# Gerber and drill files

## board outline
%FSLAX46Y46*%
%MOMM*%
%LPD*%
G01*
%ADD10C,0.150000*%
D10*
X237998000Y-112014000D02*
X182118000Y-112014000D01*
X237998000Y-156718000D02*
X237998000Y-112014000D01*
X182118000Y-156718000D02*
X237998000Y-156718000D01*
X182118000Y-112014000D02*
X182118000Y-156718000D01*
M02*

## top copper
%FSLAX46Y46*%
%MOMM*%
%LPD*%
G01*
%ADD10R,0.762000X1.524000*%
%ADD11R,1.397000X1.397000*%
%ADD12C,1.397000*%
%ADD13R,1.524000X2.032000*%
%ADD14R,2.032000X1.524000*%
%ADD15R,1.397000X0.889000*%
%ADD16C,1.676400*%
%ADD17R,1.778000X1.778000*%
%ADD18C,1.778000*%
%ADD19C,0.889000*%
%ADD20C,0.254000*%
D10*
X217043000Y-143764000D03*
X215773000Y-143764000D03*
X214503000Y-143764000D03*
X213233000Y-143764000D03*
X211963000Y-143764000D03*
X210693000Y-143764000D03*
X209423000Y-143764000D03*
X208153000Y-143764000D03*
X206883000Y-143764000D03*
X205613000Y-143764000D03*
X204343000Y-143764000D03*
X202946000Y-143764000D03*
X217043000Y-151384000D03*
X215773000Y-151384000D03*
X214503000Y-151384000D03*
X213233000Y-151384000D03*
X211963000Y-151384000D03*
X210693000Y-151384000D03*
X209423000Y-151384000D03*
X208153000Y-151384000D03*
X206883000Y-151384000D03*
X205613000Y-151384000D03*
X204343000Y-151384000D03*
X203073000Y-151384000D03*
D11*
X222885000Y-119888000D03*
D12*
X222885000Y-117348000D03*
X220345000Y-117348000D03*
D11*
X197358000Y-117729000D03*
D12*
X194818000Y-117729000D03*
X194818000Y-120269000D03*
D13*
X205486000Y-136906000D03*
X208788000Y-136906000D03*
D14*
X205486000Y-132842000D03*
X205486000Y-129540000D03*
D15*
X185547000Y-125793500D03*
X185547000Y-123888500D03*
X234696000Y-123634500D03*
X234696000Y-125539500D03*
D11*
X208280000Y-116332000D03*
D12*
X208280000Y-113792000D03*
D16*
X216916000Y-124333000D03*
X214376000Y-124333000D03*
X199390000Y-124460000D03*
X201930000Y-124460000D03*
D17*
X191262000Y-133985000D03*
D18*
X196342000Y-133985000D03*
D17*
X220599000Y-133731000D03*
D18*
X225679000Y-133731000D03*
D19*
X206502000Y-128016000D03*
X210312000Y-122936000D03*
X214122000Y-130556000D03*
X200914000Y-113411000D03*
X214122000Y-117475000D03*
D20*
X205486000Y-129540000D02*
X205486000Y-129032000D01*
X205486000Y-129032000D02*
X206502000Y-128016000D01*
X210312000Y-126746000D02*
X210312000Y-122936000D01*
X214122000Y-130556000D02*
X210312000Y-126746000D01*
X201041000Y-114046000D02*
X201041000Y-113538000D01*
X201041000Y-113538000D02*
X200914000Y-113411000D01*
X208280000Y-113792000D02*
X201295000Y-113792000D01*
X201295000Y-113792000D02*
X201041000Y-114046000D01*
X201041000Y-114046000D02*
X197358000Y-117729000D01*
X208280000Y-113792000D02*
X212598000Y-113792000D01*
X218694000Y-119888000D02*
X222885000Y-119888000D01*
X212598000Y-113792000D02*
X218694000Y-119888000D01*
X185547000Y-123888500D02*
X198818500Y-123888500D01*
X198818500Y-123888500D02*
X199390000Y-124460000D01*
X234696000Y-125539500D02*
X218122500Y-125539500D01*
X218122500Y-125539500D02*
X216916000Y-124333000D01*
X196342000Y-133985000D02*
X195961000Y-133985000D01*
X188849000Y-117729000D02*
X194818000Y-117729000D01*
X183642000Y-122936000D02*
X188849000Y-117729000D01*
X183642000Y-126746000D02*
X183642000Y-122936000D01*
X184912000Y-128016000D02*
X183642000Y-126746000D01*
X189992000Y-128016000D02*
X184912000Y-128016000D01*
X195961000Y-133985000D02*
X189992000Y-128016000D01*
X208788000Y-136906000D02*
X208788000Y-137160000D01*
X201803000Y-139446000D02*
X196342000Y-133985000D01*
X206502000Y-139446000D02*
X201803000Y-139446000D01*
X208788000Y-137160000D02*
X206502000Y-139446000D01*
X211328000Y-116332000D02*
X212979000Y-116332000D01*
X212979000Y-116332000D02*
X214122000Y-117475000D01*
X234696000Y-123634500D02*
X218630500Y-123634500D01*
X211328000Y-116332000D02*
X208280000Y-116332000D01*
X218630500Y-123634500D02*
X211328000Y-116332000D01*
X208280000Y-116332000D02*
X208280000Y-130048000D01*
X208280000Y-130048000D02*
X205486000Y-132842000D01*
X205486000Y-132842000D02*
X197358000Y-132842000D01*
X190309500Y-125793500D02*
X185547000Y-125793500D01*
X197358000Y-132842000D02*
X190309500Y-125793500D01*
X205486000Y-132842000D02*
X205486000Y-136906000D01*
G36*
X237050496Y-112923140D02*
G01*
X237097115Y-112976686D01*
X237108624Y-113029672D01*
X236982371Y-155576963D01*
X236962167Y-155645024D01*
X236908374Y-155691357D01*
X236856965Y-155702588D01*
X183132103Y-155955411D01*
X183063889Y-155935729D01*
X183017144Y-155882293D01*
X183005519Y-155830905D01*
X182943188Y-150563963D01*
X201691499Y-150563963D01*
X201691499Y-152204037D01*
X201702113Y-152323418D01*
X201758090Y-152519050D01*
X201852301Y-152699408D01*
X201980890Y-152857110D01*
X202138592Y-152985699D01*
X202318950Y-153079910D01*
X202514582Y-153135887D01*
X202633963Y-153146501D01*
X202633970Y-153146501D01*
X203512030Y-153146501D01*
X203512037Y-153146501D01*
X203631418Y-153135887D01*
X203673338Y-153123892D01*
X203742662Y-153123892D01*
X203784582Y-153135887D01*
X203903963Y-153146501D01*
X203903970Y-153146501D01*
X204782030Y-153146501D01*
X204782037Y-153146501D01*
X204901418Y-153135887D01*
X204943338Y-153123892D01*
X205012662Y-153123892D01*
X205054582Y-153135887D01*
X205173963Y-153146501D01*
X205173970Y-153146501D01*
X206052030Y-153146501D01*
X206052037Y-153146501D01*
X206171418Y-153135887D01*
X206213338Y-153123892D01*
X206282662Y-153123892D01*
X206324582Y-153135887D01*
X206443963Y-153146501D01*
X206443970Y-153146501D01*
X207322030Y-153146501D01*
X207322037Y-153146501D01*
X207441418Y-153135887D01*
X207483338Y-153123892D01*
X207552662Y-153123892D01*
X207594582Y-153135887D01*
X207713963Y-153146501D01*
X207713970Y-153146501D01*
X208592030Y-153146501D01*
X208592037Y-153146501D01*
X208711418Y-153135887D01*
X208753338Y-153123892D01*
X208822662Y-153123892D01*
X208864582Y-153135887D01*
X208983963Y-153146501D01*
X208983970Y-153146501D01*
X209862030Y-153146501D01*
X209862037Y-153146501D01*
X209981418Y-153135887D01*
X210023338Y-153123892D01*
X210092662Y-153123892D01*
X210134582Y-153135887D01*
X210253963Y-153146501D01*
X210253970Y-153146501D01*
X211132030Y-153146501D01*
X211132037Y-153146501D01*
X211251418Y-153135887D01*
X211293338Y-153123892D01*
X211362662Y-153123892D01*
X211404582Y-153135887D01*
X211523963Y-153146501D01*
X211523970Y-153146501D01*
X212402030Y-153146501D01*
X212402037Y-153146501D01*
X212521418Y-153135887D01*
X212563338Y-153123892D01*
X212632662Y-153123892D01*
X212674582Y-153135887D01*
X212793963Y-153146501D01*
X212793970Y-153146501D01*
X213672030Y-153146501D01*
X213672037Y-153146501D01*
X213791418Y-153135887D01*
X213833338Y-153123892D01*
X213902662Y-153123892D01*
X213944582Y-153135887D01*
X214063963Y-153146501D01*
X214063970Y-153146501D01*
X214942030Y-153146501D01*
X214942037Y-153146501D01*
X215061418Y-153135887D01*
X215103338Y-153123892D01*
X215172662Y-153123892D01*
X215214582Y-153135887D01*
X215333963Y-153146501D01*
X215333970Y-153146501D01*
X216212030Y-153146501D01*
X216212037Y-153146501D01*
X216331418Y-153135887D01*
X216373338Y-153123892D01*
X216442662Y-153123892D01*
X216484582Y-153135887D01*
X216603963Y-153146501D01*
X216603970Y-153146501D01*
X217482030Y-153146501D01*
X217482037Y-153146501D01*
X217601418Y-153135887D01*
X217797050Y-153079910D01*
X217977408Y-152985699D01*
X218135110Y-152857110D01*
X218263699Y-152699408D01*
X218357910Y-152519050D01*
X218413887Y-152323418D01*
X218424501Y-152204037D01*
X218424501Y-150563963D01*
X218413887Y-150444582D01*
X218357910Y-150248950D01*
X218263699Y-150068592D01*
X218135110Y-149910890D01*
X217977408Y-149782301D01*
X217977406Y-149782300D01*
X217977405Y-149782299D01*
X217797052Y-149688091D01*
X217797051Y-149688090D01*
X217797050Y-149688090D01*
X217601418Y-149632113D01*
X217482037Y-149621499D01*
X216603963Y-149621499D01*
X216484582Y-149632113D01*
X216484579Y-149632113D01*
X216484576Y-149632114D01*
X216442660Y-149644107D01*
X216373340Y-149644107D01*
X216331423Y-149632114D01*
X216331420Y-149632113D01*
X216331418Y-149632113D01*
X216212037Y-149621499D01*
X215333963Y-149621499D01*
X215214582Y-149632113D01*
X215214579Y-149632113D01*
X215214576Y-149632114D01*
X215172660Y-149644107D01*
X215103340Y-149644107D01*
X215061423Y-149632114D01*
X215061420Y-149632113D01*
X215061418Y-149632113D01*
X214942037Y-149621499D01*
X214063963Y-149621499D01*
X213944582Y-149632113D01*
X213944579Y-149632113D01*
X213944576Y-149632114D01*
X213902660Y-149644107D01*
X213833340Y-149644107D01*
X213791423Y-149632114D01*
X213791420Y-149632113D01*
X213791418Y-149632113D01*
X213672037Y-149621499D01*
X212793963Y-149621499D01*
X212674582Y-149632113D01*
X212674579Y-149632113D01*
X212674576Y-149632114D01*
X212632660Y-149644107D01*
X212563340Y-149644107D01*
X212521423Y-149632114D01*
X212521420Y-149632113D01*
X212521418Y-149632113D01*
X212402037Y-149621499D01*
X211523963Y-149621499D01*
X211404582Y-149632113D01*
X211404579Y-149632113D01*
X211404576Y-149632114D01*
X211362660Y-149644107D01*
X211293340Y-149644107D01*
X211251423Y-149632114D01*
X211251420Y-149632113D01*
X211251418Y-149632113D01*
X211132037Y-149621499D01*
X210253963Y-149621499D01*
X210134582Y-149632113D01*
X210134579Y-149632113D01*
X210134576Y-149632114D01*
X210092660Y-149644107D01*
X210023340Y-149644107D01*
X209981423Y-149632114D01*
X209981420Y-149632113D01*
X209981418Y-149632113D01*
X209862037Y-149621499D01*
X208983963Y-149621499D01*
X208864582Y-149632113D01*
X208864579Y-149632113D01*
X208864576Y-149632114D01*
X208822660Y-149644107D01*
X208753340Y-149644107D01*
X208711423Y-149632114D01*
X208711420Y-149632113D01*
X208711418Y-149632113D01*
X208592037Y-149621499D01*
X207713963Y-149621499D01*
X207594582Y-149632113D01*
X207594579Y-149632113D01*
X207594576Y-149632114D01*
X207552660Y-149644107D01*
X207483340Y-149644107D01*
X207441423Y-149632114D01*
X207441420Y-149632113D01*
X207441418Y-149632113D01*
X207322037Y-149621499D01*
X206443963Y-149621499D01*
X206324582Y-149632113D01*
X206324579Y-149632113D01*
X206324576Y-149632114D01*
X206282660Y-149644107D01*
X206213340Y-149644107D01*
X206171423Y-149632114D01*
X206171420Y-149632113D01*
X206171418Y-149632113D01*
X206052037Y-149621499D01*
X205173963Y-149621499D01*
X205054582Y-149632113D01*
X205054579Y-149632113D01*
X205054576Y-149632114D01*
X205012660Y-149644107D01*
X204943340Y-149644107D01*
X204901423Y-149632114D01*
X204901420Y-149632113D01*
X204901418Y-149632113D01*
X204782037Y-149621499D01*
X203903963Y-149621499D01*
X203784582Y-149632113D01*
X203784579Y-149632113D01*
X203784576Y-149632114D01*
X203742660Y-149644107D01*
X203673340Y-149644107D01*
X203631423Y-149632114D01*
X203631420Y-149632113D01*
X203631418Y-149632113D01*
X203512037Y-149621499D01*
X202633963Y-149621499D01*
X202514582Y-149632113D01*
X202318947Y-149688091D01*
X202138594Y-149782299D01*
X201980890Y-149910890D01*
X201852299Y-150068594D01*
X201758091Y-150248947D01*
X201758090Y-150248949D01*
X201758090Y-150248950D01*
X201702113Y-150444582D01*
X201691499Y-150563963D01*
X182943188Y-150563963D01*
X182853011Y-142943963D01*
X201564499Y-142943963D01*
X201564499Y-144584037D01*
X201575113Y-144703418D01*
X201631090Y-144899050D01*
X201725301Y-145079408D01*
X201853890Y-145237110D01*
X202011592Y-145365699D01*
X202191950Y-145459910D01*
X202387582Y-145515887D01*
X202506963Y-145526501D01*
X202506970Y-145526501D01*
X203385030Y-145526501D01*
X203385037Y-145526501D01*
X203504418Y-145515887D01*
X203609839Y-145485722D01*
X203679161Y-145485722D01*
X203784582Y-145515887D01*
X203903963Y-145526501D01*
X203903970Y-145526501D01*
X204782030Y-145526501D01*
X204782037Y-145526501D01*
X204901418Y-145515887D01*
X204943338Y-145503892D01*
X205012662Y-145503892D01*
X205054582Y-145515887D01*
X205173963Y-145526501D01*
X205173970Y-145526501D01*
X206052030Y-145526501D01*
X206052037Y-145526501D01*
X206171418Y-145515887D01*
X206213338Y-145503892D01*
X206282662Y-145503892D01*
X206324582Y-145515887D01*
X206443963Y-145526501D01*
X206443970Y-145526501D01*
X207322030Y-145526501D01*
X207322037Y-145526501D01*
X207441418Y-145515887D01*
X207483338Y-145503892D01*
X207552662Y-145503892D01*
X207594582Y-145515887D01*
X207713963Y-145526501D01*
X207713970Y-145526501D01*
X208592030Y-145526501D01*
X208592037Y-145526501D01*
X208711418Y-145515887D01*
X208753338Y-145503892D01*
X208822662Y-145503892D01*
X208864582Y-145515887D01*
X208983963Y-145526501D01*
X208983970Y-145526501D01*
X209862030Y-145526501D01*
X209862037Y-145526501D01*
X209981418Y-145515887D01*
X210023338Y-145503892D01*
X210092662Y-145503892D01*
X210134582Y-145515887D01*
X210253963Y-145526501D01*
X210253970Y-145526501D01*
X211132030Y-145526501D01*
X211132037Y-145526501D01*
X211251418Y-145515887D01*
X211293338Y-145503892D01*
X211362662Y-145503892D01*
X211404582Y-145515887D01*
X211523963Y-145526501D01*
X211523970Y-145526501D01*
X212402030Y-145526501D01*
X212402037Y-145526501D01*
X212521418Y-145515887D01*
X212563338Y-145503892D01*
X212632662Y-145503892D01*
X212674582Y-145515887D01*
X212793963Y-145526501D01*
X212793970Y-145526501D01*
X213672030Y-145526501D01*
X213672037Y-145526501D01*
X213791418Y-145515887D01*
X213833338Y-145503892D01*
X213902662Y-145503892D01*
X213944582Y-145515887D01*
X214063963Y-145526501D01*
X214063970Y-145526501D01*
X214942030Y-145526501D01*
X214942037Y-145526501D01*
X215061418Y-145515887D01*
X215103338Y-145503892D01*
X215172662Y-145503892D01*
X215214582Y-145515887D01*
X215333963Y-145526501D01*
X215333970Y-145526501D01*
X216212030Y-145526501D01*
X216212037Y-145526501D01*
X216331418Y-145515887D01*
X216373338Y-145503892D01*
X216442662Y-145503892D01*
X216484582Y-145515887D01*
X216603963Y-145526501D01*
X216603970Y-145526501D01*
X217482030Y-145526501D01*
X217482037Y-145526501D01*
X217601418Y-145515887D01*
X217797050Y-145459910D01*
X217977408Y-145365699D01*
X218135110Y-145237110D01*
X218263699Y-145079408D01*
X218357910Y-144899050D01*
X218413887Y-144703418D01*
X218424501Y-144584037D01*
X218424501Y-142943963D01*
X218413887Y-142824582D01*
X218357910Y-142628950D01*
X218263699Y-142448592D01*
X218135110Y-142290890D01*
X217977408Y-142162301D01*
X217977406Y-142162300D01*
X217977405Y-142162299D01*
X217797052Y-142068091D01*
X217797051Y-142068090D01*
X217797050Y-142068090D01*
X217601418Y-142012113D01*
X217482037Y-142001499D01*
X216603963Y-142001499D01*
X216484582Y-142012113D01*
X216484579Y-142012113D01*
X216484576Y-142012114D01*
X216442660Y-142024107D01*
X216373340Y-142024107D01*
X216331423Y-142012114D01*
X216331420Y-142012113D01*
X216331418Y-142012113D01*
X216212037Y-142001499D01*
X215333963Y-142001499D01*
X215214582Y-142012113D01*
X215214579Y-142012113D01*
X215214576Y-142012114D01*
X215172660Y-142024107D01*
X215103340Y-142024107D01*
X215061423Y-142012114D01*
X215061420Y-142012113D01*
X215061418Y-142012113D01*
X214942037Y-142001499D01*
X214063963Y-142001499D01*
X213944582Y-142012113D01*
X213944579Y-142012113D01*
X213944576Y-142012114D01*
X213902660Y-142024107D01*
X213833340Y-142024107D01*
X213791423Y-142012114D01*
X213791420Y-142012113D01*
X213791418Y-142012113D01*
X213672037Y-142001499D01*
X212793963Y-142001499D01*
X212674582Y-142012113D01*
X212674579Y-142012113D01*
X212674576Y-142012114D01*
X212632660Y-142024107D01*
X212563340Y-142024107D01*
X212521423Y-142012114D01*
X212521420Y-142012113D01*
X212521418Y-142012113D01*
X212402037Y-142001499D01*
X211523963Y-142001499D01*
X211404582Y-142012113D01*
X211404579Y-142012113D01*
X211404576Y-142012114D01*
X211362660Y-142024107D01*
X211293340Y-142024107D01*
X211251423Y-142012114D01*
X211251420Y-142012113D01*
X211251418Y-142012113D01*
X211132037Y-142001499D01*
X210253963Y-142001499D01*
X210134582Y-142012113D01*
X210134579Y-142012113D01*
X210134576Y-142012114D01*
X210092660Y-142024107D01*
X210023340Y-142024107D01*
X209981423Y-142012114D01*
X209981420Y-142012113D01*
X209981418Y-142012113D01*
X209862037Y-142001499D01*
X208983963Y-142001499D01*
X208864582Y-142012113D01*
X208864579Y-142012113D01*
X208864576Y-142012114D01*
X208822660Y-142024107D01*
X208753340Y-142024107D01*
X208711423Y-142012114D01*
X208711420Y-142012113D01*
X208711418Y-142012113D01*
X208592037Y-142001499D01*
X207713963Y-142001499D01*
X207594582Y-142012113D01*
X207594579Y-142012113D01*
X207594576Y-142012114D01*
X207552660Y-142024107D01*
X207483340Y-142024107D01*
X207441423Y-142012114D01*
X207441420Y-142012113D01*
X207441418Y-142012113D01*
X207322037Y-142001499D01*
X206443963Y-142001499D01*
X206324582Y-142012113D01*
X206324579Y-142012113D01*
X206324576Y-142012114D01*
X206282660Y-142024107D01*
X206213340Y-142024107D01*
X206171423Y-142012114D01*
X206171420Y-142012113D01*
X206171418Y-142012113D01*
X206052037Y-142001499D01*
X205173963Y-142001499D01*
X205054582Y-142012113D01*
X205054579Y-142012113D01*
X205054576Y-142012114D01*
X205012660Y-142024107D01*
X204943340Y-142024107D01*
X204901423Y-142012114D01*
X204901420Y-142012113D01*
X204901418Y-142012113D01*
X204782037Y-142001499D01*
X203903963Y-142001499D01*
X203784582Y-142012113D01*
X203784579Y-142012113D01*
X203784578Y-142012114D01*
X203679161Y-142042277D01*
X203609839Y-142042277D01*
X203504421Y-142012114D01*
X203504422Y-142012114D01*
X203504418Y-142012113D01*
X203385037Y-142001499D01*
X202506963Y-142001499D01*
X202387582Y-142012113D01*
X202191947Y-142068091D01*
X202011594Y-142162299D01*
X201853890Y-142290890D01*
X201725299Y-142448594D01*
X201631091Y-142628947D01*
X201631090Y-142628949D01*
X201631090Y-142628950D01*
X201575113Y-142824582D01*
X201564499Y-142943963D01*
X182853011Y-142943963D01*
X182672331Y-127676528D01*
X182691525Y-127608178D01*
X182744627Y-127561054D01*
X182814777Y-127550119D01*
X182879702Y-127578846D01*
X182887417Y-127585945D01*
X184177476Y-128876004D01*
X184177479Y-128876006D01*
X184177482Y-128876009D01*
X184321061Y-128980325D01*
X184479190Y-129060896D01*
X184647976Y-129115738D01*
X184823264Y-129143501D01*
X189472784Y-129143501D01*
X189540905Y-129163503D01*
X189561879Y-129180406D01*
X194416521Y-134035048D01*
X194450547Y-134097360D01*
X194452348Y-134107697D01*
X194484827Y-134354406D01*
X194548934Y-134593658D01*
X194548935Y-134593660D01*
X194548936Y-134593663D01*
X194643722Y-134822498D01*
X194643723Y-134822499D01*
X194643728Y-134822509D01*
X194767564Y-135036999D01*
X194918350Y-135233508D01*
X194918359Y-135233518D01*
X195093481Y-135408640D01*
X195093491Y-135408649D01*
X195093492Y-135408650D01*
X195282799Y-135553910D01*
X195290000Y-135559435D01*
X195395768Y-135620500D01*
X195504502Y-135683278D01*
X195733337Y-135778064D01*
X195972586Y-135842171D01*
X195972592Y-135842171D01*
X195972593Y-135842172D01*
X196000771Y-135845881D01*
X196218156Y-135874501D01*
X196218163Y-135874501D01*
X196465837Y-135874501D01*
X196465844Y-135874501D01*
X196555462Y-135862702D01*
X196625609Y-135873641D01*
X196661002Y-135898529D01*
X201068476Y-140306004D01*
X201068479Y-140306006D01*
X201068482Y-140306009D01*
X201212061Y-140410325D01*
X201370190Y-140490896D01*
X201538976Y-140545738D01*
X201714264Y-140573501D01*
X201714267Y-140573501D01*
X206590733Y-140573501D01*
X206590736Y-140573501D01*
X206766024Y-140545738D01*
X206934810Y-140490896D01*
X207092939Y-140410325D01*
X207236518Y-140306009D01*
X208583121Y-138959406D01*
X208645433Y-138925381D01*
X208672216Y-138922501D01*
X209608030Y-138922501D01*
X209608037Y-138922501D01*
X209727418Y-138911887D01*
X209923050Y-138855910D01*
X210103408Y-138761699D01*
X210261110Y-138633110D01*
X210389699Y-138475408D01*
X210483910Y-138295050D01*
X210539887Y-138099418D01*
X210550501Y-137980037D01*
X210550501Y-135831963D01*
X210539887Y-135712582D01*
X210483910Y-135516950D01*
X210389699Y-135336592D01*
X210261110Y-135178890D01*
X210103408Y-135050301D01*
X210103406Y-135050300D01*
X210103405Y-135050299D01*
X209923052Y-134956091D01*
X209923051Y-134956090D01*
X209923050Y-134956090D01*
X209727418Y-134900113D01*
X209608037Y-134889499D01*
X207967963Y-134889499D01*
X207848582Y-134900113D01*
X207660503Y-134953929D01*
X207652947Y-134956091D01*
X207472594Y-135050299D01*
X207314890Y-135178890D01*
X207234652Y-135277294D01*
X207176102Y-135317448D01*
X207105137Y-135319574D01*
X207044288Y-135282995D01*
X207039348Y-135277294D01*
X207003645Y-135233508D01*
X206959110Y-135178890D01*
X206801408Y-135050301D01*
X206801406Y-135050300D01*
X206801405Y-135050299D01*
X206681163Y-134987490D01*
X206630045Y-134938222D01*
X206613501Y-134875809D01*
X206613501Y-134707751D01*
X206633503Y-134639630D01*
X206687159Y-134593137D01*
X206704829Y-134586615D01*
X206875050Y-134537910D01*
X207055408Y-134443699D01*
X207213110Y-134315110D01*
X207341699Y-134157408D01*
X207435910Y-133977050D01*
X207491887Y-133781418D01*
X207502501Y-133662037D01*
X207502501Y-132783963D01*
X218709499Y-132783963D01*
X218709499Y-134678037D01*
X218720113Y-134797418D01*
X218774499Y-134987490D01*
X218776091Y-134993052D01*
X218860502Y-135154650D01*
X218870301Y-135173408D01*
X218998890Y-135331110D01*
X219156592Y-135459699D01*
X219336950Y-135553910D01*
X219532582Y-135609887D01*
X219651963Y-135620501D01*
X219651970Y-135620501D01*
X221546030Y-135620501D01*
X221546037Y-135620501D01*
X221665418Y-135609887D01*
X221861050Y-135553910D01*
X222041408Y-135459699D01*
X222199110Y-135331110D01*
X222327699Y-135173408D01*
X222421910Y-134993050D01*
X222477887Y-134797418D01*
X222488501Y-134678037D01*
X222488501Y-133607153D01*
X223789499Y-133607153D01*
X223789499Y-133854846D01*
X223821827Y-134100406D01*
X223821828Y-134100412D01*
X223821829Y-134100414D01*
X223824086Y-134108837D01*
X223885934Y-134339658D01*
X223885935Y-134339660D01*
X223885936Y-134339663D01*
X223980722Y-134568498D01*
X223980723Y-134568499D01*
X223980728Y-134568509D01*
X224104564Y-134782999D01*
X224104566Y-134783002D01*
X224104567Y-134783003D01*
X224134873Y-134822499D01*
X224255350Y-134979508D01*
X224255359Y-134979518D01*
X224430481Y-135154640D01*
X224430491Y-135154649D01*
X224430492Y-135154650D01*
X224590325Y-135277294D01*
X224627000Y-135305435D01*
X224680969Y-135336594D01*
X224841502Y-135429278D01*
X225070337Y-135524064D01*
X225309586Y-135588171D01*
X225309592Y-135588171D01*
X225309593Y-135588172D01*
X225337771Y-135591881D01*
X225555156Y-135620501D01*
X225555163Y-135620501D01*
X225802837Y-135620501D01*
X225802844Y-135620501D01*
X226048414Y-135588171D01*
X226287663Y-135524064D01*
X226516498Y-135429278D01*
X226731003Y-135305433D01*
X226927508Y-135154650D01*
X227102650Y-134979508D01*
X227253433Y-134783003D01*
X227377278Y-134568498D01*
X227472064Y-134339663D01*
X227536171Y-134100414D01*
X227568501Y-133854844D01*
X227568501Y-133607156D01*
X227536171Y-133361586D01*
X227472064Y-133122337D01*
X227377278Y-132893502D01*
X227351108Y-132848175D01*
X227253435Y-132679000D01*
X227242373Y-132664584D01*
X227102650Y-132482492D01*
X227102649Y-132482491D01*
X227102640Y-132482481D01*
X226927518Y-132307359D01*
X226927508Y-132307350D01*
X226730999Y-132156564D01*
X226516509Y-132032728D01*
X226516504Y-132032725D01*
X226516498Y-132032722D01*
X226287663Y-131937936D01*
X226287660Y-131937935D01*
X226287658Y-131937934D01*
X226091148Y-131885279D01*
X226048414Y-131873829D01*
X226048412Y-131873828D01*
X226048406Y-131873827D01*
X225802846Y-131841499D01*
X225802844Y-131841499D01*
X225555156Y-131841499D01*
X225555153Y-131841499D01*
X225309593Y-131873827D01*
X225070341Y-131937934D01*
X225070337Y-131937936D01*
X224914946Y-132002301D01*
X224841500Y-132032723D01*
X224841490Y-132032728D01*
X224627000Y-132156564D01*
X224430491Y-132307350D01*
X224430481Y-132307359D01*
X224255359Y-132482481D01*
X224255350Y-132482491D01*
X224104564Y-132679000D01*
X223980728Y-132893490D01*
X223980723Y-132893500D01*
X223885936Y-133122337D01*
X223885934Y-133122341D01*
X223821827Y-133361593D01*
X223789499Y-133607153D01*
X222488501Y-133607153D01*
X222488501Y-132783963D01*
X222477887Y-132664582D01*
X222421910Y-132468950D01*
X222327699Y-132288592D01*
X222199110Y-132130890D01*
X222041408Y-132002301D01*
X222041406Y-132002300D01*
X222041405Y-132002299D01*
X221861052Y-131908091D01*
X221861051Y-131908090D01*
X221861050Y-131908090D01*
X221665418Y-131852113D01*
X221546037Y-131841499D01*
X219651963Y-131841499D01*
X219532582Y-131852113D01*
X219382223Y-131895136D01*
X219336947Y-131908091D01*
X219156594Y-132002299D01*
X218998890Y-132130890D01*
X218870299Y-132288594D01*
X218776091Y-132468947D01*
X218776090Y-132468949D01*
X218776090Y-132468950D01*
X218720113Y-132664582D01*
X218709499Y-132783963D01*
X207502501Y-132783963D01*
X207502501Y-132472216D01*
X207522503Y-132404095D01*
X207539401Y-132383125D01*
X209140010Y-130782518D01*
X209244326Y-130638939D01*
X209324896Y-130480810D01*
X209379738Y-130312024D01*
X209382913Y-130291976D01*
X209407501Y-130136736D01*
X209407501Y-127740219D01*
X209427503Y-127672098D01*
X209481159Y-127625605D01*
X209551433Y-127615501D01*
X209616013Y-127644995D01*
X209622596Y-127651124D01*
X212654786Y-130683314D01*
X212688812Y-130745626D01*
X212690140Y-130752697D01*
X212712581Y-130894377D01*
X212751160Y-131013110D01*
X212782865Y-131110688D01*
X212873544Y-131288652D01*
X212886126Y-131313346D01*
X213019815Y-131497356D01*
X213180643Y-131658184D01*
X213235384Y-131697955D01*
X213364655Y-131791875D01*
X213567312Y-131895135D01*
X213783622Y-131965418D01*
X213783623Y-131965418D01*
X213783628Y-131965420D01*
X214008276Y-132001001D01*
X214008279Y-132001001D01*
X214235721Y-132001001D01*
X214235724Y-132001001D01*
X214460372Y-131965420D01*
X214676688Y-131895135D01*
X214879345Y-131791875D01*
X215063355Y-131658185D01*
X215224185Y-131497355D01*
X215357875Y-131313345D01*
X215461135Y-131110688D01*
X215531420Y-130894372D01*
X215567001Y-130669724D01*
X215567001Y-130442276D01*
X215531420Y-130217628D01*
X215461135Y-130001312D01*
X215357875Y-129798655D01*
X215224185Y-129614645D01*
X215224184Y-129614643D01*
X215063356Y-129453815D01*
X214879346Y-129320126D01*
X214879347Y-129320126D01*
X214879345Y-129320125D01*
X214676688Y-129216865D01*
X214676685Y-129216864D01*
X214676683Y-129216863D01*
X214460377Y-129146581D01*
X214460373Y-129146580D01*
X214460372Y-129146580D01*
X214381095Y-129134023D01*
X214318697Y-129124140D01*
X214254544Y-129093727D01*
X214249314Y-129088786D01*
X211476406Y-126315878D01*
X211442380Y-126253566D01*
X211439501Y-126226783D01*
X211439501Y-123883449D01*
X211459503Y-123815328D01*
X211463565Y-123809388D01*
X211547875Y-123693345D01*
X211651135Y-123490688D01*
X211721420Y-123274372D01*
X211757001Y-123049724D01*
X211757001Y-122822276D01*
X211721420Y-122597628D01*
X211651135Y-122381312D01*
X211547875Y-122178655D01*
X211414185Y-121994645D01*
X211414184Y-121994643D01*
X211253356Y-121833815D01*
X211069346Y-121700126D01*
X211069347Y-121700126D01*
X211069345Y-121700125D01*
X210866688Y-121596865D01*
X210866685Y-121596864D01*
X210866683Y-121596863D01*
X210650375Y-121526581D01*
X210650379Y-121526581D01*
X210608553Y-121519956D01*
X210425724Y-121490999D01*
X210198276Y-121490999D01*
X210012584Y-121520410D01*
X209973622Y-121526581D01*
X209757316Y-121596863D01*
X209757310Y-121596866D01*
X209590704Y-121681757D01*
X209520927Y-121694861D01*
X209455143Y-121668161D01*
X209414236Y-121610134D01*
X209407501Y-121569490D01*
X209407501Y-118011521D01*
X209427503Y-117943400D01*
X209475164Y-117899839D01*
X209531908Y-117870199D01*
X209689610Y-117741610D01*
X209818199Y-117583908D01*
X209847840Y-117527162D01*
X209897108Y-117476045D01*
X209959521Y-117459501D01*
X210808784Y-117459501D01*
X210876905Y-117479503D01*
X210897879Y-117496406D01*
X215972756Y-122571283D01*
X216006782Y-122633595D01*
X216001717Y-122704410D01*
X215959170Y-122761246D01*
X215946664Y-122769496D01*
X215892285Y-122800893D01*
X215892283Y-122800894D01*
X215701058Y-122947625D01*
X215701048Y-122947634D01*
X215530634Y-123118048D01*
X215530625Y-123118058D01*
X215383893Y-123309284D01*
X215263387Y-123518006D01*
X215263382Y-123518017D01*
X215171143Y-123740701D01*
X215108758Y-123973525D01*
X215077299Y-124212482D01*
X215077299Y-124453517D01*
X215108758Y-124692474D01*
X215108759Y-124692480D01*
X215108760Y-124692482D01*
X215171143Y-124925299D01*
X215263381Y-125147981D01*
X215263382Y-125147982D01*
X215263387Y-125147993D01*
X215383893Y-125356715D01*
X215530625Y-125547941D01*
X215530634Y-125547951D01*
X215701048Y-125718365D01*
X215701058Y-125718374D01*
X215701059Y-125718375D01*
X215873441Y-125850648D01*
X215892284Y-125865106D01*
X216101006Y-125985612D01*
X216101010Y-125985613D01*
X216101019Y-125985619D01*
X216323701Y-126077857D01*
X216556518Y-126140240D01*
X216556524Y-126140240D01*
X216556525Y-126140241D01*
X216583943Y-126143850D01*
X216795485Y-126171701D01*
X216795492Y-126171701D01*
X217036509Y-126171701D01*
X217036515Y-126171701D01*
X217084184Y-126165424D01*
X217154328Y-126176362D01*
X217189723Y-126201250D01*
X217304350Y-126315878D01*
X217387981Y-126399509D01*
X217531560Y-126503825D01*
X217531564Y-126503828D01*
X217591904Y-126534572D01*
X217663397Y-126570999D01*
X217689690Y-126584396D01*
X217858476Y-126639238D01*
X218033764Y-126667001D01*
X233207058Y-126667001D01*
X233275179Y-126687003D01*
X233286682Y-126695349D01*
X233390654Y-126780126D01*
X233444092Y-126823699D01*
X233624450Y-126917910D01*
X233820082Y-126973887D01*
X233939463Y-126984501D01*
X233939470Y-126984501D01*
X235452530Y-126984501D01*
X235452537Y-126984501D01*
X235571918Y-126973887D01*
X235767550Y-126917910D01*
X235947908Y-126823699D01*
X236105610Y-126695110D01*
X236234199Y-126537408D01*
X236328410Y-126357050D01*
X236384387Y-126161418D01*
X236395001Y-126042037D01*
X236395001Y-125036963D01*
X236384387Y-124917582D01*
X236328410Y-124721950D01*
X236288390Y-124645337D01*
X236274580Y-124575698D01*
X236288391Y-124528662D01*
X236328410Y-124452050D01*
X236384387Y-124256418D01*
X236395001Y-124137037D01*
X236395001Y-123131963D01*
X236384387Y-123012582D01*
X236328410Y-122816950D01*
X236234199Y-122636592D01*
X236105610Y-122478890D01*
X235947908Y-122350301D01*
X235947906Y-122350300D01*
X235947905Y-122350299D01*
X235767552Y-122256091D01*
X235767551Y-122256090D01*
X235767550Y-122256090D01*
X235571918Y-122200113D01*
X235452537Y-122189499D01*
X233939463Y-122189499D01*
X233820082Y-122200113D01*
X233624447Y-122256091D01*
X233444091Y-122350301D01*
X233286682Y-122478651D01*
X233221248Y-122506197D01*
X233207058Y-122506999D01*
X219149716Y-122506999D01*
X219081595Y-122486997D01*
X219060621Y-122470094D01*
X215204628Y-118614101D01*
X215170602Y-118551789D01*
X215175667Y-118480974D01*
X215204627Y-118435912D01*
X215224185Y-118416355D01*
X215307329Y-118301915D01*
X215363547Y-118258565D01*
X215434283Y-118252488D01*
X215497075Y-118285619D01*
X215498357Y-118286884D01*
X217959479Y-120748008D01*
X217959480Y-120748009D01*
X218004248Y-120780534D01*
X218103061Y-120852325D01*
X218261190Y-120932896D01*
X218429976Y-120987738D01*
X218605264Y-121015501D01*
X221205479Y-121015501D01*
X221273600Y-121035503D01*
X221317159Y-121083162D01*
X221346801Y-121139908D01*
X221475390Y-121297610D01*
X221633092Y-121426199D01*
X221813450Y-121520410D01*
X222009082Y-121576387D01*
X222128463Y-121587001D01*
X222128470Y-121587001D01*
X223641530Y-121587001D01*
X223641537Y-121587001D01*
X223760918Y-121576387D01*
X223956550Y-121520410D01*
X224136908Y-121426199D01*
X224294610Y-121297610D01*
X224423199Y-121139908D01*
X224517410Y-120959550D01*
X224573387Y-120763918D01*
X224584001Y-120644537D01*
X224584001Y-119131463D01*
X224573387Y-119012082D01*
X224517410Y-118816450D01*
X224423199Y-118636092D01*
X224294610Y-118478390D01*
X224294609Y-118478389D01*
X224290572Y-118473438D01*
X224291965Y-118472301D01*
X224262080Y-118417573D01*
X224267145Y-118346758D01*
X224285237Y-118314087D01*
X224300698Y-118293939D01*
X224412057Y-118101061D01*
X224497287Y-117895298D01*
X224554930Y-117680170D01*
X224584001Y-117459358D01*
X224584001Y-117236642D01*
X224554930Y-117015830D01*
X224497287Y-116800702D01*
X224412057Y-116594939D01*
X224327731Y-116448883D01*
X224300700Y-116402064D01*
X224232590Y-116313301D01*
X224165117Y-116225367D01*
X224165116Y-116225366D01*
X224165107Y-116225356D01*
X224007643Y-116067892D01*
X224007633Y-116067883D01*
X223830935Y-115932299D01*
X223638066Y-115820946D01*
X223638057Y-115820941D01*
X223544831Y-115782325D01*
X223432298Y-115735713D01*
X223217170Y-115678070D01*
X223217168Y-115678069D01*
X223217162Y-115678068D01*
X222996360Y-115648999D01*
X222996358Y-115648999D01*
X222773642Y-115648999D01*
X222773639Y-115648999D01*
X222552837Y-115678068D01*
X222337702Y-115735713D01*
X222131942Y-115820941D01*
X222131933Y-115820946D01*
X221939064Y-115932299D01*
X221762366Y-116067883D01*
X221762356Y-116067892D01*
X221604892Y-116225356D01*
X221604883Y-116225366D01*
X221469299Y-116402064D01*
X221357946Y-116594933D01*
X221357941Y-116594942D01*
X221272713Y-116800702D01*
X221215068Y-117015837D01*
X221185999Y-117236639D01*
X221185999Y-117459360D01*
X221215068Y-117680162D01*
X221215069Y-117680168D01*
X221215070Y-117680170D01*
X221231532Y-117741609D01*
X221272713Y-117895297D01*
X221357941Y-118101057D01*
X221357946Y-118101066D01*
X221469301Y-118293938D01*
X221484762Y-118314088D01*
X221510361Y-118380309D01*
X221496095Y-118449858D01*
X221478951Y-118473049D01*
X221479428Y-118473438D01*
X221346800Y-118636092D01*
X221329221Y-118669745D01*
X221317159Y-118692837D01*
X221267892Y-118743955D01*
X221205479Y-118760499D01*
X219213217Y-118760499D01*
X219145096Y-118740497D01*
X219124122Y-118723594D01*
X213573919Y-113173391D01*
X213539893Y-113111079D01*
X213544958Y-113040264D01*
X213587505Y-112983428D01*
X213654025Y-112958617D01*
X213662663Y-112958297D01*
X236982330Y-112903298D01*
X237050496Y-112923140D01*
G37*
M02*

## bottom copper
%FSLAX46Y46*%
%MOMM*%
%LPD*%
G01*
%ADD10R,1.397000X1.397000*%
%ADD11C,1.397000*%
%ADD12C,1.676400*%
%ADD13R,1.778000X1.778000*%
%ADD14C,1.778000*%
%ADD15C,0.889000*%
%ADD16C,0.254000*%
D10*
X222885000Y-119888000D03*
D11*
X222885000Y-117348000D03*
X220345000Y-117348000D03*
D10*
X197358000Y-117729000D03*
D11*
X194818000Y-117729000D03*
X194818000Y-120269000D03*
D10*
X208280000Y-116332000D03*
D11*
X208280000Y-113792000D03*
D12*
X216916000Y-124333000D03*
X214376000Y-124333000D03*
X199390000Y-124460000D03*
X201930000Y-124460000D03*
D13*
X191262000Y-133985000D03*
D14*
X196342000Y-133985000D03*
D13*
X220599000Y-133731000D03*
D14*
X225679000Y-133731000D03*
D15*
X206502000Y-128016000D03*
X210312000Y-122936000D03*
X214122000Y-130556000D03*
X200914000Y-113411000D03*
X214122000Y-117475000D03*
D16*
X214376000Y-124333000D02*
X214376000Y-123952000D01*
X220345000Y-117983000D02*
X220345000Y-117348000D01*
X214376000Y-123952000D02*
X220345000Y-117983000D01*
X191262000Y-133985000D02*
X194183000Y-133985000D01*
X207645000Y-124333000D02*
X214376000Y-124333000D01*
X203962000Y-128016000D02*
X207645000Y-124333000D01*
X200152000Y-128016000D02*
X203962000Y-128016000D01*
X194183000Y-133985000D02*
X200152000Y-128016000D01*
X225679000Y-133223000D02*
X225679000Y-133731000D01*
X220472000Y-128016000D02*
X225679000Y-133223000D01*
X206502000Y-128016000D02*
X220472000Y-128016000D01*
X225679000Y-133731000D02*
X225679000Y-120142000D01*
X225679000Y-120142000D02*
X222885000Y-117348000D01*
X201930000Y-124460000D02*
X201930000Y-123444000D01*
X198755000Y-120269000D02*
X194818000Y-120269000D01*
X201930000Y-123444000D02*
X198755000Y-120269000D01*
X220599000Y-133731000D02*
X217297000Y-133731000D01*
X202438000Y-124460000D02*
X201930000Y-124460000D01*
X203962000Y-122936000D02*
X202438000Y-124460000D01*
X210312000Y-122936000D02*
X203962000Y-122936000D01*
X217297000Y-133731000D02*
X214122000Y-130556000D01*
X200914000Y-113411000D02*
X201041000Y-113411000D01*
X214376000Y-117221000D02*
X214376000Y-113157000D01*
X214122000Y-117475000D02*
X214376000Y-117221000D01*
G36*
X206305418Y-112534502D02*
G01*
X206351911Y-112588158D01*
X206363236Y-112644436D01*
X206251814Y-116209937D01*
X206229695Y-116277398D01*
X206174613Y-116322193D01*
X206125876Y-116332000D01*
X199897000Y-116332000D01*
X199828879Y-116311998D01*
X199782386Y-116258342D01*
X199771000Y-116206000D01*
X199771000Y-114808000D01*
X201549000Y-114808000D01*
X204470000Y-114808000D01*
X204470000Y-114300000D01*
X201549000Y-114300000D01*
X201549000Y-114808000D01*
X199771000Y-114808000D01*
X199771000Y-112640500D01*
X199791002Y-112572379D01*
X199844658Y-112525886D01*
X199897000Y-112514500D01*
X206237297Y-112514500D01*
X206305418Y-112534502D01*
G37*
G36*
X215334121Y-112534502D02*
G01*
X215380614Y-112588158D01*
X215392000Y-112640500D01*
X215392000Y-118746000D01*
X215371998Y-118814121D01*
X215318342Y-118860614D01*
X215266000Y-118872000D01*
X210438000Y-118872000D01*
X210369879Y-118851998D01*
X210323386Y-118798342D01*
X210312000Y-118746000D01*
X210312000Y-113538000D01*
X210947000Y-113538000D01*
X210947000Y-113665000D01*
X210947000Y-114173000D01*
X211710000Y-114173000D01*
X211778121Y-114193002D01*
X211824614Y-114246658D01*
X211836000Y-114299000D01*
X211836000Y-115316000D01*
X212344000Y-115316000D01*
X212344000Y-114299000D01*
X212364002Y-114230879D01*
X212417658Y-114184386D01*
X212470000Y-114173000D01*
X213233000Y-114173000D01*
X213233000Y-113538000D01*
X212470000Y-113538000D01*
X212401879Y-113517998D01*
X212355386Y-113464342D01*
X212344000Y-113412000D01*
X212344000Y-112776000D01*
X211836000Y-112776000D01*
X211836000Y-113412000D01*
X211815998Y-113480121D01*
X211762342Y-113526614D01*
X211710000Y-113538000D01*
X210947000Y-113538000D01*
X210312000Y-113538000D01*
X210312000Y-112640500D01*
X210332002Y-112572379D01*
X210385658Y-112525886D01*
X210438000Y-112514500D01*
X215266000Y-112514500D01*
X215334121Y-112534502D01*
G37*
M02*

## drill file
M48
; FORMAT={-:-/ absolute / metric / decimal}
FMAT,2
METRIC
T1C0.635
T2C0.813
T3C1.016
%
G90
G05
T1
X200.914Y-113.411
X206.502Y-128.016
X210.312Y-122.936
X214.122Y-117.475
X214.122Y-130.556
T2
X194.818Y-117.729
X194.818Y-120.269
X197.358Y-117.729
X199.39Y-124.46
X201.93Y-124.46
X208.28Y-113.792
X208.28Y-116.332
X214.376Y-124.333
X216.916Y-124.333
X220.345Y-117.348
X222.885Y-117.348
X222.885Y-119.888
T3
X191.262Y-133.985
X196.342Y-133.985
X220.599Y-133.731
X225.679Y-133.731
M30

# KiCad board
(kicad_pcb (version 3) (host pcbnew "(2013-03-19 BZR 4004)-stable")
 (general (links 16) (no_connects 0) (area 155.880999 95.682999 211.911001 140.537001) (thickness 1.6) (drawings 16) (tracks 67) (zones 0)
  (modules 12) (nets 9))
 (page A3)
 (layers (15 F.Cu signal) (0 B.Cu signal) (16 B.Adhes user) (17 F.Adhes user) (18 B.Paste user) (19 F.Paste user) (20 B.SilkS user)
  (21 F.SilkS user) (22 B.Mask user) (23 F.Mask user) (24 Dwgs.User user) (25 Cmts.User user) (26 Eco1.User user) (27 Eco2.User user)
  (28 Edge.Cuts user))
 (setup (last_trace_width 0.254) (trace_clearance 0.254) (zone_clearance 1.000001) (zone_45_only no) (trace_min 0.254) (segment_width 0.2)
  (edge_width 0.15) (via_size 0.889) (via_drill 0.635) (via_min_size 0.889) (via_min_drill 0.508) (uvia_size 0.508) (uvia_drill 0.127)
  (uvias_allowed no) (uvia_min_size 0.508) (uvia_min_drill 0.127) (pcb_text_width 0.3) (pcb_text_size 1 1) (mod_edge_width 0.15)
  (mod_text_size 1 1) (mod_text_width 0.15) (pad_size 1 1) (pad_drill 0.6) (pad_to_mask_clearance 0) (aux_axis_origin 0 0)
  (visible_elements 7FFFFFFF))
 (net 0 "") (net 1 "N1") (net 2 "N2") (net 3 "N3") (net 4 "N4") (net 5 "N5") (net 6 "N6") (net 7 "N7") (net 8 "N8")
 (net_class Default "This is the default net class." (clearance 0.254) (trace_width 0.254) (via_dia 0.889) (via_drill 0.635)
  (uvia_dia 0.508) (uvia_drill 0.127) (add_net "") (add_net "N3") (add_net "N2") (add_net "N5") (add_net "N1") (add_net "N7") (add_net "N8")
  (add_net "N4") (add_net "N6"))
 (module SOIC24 (layer F.Cu) (at 210.058 147.574 180)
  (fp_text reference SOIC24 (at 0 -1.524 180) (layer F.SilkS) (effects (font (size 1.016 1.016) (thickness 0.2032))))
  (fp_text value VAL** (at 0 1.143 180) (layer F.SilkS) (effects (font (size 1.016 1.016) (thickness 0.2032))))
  (pad 1 smd rect (at -6.985 3.81 180) (size 0.762 1.524) (layers F.Cu F.Paste F.Mask))
  (pad 2 smd rect (at -5.715 3.81 180) (size 0.762 1.524) (layers F.Cu F.Paste F.Mask))
  (pad 3 smd rect (at -4.445 3.81 180) (size 0.762 1.524) (layers F.Cu F.Paste F.Mask))
  (pad 4 smd rect (at -3.175 3.81 180) (size 0.762 1.524) (layers F.Cu F.Paste F.Mask))
  (pad 5 smd rect (at -1.905 3.81 180) (size 0.762 1.524) (layers F.Cu F.Paste F.Mask))
  (pad 6 smd rect (at -0.635 3.81 180) (size 0.762 1.524) (layers F.Cu F.Paste F.Mask))
  (pad 7 smd rect (at 0.635 3.81 180) (size 0.762 1.524) (layers F.Cu F.Paste F.Mask))
  (pad 8 smd rect (at 1.905 3.81 180) (size 0.762 1.524) (layers F.Cu F.Paste F.Mask))
  (pad 9 smd rect (at 3.175 3.81 180) (size 0.762 1.524) (layers F.Cu F.Paste F.Mask))
  (pad 10 smd rect (at 4.445 3.81 180) (size 0.762 1.524) (layers F.Cu F.Paste F.Mask))
  (pad 11 smd rect (at 5.715 3.81 180) (size 0.762 1.524) (layers F.Cu F.Paste F.Mask))
  (pad 12 smd rect (at 7.112 3.81 180) (size 0.762 1.524) (layers F.Cu F.Paste F.Mask))
  (pad 24 smd rect (at -6.985 -3.81 180) (size 0.762 1.524) (layers F.Cu F.Paste F.Mask))
  (pad 23 smd rect (at -5.715 -3.81 180) (size 0.762 1.524) (layers F.Cu F.Paste F.Mask))
  (pad 22 smd rect (at -4.445 -3.81 180) (size 0.762 1.524) (layers F.Cu F.Paste F.Mask))
  (pad 21 smd rect (at -3.175 -3.81 180) (size 0.762 1.524) (layers F.Cu F.Paste F.Mask))
  (pad 20 smd rect (at -1.905 -3.81 180) (size 0.762 1.524) (layers F.Cu F.Paste F.Mask))
  (pad 19 smd rect (at -0.635 -3.81 180) (size 0.762 1.524) (layers F.Cu F.Paste F.Mask))
  (pad 18 smd rect (at 0.635 -3.81 180) (size 0.762 1.524) (layers F.Cu F.Paste F.Mask))
  (pad 17 smd rect (at 1.905 -3.81 180) (size 0.762 1.524) (layers F.Cu F.Paste F.Mask))
  (pad 16 smd rect (at 3.175 -3.81 180) (size 0.762 1.524) (layers F.Cu F.Paste F.Mask))
  (pad 15 smd rect (at 4.445 -3.81 180) (size 0.762 1.524) (layers F.Cu F.Paste F.Mask))
  (pad 14 smd rect (at 5.715 -3.81 180) (size 0.762 1.524) (layers F.Cu F.Paste F.Mask))
  (pad 13 smd rect (at 6.985 -3.81 180) (size 0.762 1.524) (layers F.Cu F.Paste F.Mask)))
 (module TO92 (layer F.Cu) (at 221.615 118.618 270) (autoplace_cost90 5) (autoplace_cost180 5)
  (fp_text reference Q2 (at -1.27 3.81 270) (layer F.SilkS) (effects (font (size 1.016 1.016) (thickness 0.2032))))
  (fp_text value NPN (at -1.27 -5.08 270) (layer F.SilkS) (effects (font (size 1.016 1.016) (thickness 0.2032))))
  (pad 1 thru_hole rect (at 1.27 -1.27 270) (size 1.397 1.397) (drill 0.8128) (layers *.Cu *.Mask F.SilkS) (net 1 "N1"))
  (pad 2 thru_hole circle (at -1.27 -1.27 270) (size 1.397 1.397) (drill 0.8128) (layers *.Cu *.Mask F.SilkS) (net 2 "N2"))
  (pad 3 thru_hole circle (at -1.27 1.27 270) (size 1.397 1.397) (drill 0.8128) (layers *.Cu *.Mask F.SilkS) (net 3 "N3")))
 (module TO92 (layer F.Cu) (at 196.088 118.999)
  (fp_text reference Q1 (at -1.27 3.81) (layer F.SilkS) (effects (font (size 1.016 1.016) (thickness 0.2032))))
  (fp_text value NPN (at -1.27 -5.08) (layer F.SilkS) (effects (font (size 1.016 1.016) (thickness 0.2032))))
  (pad 1 thru_hole rect (at 1.27 -1.27) (size 1.397 1.397) (drill 0.8128) (layers *.Cu *.Mask F.SilkS) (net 1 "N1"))
  (pad 2 thru_hole circle (at -1.27 -1.27) (size 1.397 1.397) (drill 0.8128) (layers *.Cu *.Mask F.SilkS) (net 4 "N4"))
  (pad 3 thru_hole circle (at -1.27 1.27) (size 1.397 1.397) (drill 0.8128) (layers *.Cu *.Mask F.SilkS) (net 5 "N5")))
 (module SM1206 (layer F.Cu) (at 207.137 136.906)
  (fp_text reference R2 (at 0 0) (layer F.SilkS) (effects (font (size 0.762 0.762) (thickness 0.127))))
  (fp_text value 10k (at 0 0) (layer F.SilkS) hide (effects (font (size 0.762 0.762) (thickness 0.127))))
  (pad 1 smd rect (at -1.651 0) (size 1.524 2.032) (layers F.Cu F.Paste F.Mask) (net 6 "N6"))
  (pad 2 smd rect (at 1.651 0) (size 1.524 2.032) (layers F.Cu F.Paste F.Mask) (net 4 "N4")))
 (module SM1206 (layer F.Cu) (at 205.486 131.191 90)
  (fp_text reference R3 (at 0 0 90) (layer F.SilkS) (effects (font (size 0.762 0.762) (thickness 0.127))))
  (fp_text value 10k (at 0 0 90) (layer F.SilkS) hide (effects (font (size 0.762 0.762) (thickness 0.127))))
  (pad 1 smd rect (at -1.651 0 90) (size 1.524 2.032) (layers F.Cu F.Paste F.Mask) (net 6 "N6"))
  (pad 2 smd rect (at 1.651 0 90) (size 1.524 2.032) (layers F.Cu F.Paste F.Mask) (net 2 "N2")))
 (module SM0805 (layer F.Cu) (at 185.547 124.841 90)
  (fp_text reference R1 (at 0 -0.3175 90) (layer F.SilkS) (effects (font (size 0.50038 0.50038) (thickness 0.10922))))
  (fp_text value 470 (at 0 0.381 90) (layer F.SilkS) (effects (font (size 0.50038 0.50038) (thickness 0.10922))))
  (pad 1 smd rect (at -0.9525 0 90) (size 0.889 1.397) (layers F.Cu F.Paste F.Mask) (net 6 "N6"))
  (pad 2 smd rect (at 0.9525 0 90) (size 0.889 1.397) (layers F.Cu F.Paste F.Mask) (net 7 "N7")))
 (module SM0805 (layer F.Cu) (at 234.696 124.587 270)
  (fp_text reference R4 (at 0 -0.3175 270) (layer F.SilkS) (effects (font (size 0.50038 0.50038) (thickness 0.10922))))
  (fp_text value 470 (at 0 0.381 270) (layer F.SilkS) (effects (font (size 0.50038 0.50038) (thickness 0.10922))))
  (pad 1 smd rect (at -0.9525 0 270) (size 0.889 1.397) (layers F.Cu F.Paste F.Mask) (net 6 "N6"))
  (pad 2 smd rect (at 0.9525 0 270) (size 0.889 1.397) (layers F.Cu F.Paste F.Mask) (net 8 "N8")))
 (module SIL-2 (layer F.Cu) (at 208.28 115.062 90)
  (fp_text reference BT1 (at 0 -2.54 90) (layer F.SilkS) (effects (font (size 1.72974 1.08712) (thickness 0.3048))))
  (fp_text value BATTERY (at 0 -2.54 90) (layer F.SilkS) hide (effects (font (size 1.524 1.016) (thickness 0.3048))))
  (pad 1 thru_hole rect (at -1.27 0 90) (size 1.397 1.397) (drill 0.8128) (layers *.Cu *.Mask F.SilkS) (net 6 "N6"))
  (pad 2 thru_hole circle (at 1.27 0 90) (size 1.397 1.397) (drill 0.8128) (layers *.Cu *.Mask F.SilkS) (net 1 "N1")))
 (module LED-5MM (layer F.Cu) (at 215.646 124.333 180)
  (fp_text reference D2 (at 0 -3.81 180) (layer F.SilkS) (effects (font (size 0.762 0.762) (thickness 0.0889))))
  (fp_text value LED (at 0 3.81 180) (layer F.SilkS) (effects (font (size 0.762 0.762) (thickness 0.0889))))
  (pad 1 thru_hole circle (at -1.27 0 180) (size 1.6764 1.6764) (drill 0.8128) (layers *.Cu *.Mask F.SilkS) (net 8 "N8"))
  (pad 2 thru_hole circle (at 1.27 0 180) (size 1.6764 1.6764) (drill 0.8128) (layers *.Cu *.Mask F.SilkS) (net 3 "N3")))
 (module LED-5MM (layer F.Cu) (at 200.66 124.46)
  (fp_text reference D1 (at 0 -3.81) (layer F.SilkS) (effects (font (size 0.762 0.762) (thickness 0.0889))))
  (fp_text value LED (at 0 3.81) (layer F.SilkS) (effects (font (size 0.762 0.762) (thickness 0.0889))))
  (pad 1 thru_hole circle (at -1.27 0) (size 1.6764 1.6764) (drill 0.8128) (layers *.Cu *.Mask F.SilkS) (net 7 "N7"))
  (pad 2 thru_hole circle (at 1.27 0) (size 1.6764 1.6764) (drill 0.8128) (layers *.Cu *.Mask F.SilkS) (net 5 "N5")))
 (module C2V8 (layer F.Cu) (at 193.802 133.985)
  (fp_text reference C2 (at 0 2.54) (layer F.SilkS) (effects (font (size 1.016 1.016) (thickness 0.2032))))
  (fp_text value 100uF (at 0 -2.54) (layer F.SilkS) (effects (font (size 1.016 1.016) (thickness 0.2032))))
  (pad 1 thru_hole rect (at -2.54 0) (size 1.778 1.778) (drill 1.016) (layers *.Cu *.Mask F.SilkS) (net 3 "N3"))
  (pad 2 thru_hole circle (at 2.54 0) (size 1.778 1.778) (drill 1.016) (layers *.Cu *.Mask F.SilkS) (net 4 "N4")))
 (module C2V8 (layer F.Cu) (at 223.139 133.731)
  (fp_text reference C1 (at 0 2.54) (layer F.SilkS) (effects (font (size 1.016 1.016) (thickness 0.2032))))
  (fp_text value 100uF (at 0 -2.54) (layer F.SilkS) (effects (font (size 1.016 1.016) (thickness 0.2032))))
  (pad 1 thru_hole rect (at -2.54 0) (size 1.778 1.778) (drill 1.016) (layers *.Cu *.Mask F.SilkS) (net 5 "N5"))
  (pad 2 thru_hole circle (at 2.54 0) (size 1.778 1.778) (drill 1.016) (layers *.Cu *.Mask F.SilkS) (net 2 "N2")))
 (gr_line (start 237.998 112.014) (end 182.118 112.014) (angle 90) (layer Edge.Cuts) (width 0.15))
 (gr_line (start 237.998 156.718) (end 237.998 112.014) (angle 90) (layer Edge.Cuts) (width 0.15))
 (gr_line (start 182.118 156.718) (end 237.998 156.718) (angle 90) (layer Edge.Cuts) (width 0.15))
 (gr_line (start 182.118 112.014) (end 182.118 156.718) (angle 90) (layer Edge.Cuts) (width 0.15))
 (segment (start 214.376 124.333) (end 214.376 123.952) (width 0.254) (layer B.Cu) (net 3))
 (segment (start 220.345 117.983) (end 220.345 117.348) (width 0.254) (layer B.Cu) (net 3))
 (segment (start 214.376 123.952) (end 220.345 117.983) (width 0.254) (layer B.Cu) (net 3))
 (segment (start 191.262 133.985) (end 194.183 133.985) (width 0.254) (layer B.Cu) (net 3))
 (segment (start 207.645 124.333) (end 214.376 124.333) (width 0.254) (layer B.Cu) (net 3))
 (segment (start 203.962 128.016) (end 207.645 124.333) (width 0.254) (layer B.Cu) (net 3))
 (segment (start 200.152 128.016) (end 203.962 128.016) (width 0.254) (layer B.Cu) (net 3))
 (segment (start 194.183 133.985) (end 200.152 128.016) (width 0.254) (layer B.Cu) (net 3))
 (segment (start 205.486 129.54) (end 205.486 129.032) (width 0.254) (layer F.Cu) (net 2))
 (segment (start 225.679 133.223) (end 225.679 133.731) (width 0.254) (layer B.Cu) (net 2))
 (segment (start 220.472 128.016) (end 225.679 133.223) (width 0.254) (layer B.Cu) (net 2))
 (segment (start 206.502 128.016) (end 220.472 128.016) (width 0.254) (layer B.Cu) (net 2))
 (via (at 206.502 128.016) (size 0.889) (layers F.Cu B.Cu) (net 2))
 (segment (start 205.486 129.032) (end 206.502 128.016) (width 0.254) (layer F.Cu) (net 2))
 (segment (start 225.679 133.731) (end 225.679 120.142) (width 0.254) (layer B.Cu) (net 2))
 (segment (start 225.679 120.142) (end 222.885 117.348) (width 0.254) (layer B.Cu) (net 2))
 (segment (start 201.93 124.46) (end 201.93 123.444) (width 0.254) (layer B.Cu) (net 5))
 (segment (start 198.755 120.269) (end 194.818 120.269) (width 0.254) (layer B.Cu) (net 5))
 (segment (start 201.93 123.444) (end 198.755 120.269) (width 0.254) (layer B.Cu) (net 5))
 (segment (start 220.599 133.731) (end 217.297 133.731) (width 0.254) (layer B.Cu) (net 5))
 (segment (start 202.438 124.46) (end 201.93 124.46) (width 0.254) (layer B.Cu) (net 5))
 (segment (start 203.962 122.936) (end 202.438 124.46) (width 0.254) (layer B.Cu) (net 5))
 (segment (start 210.312 122.936) (end 203.962 122.936) (width 0.254) (layer B.Cu) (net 5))
 (via (at 210.312 122.936) (size 0.889) (layers F.Cu B.Cu) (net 5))
 (segment (start 210.312 126.746) (end 210.312 122.936) (width 0.254) (layer F.Cu) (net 5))
 (segment (start 214.122 130.556) (end 210.312 126.746) (width 0.254) (layer F.Cu) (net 5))
 (via (at 214.122 130.556) (size 0.889) (layers F.Cu B.Cu) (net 5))
 (segment (start 217.297 133.731) (end 214.122 130.556) (width 0.254) (layer B.Cu) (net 5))
 (segment (start 201.041 114.046) (end 201.041 113.538) (width 0.254) (layer F.Cu) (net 1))
 (segment (start 200.914 113.411) (end 201.041 113.411) (width 0.254) (layer B.Cu) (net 1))
 (via (at 200.914 113.411) (size 0.889) (layers F.Cu B.Cu) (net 1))
 (segment (start 201.041 113.538) (end 200.914 113.411) (width 0.254) (layer F.Cu) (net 1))
 (segment (start 208.28 113.792) (end 201.295 113.792) (width 0.254) (layer F.Cu) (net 1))
 (segment (start 201.295 113.792) (end 201.041 114.046) (width 0.254) (layer F.Cu) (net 1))
 (segment (start 201.041 114.046) (end 197.358 117.729) (width 0.254) (layer F.Cu) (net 1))
 (segment (start 208.28 113.792) (end 212.598 113.792) (width 0.254) (layer F.Cu) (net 1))
 (segment (start 218.694 119.888) (end 222.885 119.888) (width 0.254) (layer F.Cu) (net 1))
 (segment (start 212.598 113.792) (end 218.694 119.888) (width 0.254) (layer F.Cu) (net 1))
 (segment (start 185.547 123.8885) (end 198.8185 123.8885) (width 0.254) (layer F.Cu) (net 7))
 (segment (start 198.8185 123.8885) (end 199.39 124.46) (width 0.254) (layer F.Cu) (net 7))
 (segment (start 234.696 125.5395) (end 218.1225 125.5395) (width 0.254) (layer F.Cu) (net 8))
 (segment (start 218.1225 125.5395) (end 216.916 124.333) (width 0.254) (layer F.Cu) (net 8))
 (segment (start 196.342 133.985) (end 195.961 133.985) (width 0.254) (layer F.Cu) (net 4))
 (segment (start 188.849 117.729) (end 194.818 117.729) (width 0.254) (layer F.Cu) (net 4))
 (segment (start 183.642 122.936) (end 188.849 117.729) (width 0.254) (layer F.Cu) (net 4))
 (segment (start 183.642 126.746) (end 183.642 122.936) (width 0.254) (layer F.Cu) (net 4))
 (segment (start 184.912 128.016) (end 183.642 126.746) (width 0.254) (layer F.Cu) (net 4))
 (segment (start 189.992 128.016) (end 184.912 128.016) (width 0.254) (layer F.Cu) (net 4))
 (segment (start 195.961 133.985) (end 189.992 128.016) (width 0.254) (layer F.Cu) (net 4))
 (segment (start 208.788 136.906) (end 208.788 137.16) (width 0.254) (layer F.Cu) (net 4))
 (segment (start 201.803 139.446) (end 196.342 133.985) (width 0.254) (layer F.Cu) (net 4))
 (segment (start 206.502 139.446) (end 201.803 139.446) (width 0.254) (layer F.Cu) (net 4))
 (segment (start 208.788 137.16) (end 206.502 139.446) (width 0.254) (layer F.Cu) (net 4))
 (segment (start 211.328 116.332) (end 212.979 116.332) (width 0.254) (layer F.Cu) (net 6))
 (segment (start 214.376 117.221) (end 214.376 113.157) (width 0.254) (layer B.Cu) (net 6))
 (segment (start 214.122 117.475) (end 214.376 117.221) (width 0.254) (layer B.Cu) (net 6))
 (via (at 214.122 117.475) (size 0.889) (layers F.Cu B.Cu) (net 6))
 (segment (start 212.979 116.332) (end 214.122 117.475) (width 0.254) (layer F.Cu) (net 6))
 (segment (start 234.696 123.6345) (end 218.6305 123.6345) (width 0.254) (layer F.Cu) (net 6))
 (segment (start 211.328 116.332) (end 208.28 116.332) (width 0.254) (layer F.Cu) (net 6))
 (segment (start 218.6305 123.6345) (end 211.328 116.332) (width 0.254) (layer F.Cu) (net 6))
 (segment (start 208.28 116.332) (end 208.28 130.048) (width 0.254) (layer F.Cu) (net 6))
 (segment (start 208.28 130.048) (end 205.486 132.842) (width 0.254) (layer F.Cu) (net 6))
 (segment (start 205.486 132.842) (end 197.358 132.842) (width 0.254) (layer F.Cu) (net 6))
 (segment (start 190.3095 125.7935) (end 185.547 125.7935) (width 0.254) (layer F.Cu) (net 6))
 (segment (start 197.358 132.842) (end 190.3095 125.7935) (width 0.254) (layer F.Cu) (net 6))
 (segment (start 205.486 132.842) (end 205.486 136.906) (width 0.254) (layer F.Cu) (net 6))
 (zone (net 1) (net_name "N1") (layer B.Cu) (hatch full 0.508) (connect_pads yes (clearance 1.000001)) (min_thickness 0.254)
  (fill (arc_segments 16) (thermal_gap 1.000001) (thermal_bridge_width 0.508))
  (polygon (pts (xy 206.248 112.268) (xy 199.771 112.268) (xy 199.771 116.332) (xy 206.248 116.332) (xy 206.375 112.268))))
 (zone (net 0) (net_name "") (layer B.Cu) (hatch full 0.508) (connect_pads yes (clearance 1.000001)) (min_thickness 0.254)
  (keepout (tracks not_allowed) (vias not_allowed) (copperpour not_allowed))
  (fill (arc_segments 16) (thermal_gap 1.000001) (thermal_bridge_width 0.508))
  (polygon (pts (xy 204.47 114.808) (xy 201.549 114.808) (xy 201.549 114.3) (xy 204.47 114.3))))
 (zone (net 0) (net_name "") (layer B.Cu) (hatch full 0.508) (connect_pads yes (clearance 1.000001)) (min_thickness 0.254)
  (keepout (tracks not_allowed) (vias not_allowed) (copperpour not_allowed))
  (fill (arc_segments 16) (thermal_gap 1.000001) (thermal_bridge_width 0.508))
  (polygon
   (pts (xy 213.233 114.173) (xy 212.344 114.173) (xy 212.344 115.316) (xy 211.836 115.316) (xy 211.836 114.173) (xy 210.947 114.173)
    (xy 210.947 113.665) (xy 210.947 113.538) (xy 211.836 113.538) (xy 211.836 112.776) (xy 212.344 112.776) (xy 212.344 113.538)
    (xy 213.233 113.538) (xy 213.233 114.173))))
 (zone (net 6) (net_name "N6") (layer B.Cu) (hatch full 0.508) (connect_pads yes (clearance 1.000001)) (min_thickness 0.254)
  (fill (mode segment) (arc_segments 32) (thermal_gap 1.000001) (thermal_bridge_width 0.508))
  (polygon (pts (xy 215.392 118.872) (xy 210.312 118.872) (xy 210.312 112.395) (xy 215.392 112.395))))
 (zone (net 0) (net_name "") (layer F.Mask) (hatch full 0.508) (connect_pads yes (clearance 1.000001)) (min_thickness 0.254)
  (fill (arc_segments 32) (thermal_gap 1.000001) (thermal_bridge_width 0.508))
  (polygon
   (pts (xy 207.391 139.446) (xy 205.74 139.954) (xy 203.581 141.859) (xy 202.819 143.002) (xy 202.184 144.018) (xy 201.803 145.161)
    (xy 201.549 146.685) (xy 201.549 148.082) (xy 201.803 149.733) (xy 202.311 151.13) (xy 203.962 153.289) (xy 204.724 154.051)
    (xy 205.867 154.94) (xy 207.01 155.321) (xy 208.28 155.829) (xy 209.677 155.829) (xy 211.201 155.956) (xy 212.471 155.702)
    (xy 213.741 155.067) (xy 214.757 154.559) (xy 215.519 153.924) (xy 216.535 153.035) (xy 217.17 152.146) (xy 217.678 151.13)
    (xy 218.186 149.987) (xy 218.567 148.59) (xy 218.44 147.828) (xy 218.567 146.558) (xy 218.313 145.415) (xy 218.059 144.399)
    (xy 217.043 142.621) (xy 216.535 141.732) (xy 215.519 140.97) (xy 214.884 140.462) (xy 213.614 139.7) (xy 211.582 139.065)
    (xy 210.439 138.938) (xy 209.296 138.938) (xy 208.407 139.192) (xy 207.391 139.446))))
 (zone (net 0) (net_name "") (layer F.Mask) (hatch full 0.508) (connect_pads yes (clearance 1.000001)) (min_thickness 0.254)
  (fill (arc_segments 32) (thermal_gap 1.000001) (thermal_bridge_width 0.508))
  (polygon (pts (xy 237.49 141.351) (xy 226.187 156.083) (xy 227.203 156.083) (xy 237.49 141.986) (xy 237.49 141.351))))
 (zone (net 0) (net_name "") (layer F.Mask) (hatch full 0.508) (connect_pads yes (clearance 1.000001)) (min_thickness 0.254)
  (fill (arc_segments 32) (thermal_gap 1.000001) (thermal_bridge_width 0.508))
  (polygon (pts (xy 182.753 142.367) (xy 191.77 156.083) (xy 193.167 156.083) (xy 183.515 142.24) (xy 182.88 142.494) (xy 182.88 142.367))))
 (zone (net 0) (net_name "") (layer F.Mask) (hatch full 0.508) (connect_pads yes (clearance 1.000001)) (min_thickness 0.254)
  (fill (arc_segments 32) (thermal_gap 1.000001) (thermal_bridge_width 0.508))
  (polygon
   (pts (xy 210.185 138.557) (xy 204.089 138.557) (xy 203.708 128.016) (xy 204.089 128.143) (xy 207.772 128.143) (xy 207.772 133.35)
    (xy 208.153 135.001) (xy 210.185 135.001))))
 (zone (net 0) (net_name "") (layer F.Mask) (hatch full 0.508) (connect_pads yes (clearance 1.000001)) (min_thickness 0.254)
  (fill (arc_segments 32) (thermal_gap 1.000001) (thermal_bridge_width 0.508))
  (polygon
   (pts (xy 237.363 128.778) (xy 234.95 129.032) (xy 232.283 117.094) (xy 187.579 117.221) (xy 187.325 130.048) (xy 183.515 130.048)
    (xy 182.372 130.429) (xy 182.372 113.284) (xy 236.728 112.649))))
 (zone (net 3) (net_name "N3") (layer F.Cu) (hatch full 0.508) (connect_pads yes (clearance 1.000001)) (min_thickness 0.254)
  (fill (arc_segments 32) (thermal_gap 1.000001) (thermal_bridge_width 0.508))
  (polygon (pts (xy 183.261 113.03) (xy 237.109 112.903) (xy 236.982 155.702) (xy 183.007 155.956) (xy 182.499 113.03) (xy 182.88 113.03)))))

